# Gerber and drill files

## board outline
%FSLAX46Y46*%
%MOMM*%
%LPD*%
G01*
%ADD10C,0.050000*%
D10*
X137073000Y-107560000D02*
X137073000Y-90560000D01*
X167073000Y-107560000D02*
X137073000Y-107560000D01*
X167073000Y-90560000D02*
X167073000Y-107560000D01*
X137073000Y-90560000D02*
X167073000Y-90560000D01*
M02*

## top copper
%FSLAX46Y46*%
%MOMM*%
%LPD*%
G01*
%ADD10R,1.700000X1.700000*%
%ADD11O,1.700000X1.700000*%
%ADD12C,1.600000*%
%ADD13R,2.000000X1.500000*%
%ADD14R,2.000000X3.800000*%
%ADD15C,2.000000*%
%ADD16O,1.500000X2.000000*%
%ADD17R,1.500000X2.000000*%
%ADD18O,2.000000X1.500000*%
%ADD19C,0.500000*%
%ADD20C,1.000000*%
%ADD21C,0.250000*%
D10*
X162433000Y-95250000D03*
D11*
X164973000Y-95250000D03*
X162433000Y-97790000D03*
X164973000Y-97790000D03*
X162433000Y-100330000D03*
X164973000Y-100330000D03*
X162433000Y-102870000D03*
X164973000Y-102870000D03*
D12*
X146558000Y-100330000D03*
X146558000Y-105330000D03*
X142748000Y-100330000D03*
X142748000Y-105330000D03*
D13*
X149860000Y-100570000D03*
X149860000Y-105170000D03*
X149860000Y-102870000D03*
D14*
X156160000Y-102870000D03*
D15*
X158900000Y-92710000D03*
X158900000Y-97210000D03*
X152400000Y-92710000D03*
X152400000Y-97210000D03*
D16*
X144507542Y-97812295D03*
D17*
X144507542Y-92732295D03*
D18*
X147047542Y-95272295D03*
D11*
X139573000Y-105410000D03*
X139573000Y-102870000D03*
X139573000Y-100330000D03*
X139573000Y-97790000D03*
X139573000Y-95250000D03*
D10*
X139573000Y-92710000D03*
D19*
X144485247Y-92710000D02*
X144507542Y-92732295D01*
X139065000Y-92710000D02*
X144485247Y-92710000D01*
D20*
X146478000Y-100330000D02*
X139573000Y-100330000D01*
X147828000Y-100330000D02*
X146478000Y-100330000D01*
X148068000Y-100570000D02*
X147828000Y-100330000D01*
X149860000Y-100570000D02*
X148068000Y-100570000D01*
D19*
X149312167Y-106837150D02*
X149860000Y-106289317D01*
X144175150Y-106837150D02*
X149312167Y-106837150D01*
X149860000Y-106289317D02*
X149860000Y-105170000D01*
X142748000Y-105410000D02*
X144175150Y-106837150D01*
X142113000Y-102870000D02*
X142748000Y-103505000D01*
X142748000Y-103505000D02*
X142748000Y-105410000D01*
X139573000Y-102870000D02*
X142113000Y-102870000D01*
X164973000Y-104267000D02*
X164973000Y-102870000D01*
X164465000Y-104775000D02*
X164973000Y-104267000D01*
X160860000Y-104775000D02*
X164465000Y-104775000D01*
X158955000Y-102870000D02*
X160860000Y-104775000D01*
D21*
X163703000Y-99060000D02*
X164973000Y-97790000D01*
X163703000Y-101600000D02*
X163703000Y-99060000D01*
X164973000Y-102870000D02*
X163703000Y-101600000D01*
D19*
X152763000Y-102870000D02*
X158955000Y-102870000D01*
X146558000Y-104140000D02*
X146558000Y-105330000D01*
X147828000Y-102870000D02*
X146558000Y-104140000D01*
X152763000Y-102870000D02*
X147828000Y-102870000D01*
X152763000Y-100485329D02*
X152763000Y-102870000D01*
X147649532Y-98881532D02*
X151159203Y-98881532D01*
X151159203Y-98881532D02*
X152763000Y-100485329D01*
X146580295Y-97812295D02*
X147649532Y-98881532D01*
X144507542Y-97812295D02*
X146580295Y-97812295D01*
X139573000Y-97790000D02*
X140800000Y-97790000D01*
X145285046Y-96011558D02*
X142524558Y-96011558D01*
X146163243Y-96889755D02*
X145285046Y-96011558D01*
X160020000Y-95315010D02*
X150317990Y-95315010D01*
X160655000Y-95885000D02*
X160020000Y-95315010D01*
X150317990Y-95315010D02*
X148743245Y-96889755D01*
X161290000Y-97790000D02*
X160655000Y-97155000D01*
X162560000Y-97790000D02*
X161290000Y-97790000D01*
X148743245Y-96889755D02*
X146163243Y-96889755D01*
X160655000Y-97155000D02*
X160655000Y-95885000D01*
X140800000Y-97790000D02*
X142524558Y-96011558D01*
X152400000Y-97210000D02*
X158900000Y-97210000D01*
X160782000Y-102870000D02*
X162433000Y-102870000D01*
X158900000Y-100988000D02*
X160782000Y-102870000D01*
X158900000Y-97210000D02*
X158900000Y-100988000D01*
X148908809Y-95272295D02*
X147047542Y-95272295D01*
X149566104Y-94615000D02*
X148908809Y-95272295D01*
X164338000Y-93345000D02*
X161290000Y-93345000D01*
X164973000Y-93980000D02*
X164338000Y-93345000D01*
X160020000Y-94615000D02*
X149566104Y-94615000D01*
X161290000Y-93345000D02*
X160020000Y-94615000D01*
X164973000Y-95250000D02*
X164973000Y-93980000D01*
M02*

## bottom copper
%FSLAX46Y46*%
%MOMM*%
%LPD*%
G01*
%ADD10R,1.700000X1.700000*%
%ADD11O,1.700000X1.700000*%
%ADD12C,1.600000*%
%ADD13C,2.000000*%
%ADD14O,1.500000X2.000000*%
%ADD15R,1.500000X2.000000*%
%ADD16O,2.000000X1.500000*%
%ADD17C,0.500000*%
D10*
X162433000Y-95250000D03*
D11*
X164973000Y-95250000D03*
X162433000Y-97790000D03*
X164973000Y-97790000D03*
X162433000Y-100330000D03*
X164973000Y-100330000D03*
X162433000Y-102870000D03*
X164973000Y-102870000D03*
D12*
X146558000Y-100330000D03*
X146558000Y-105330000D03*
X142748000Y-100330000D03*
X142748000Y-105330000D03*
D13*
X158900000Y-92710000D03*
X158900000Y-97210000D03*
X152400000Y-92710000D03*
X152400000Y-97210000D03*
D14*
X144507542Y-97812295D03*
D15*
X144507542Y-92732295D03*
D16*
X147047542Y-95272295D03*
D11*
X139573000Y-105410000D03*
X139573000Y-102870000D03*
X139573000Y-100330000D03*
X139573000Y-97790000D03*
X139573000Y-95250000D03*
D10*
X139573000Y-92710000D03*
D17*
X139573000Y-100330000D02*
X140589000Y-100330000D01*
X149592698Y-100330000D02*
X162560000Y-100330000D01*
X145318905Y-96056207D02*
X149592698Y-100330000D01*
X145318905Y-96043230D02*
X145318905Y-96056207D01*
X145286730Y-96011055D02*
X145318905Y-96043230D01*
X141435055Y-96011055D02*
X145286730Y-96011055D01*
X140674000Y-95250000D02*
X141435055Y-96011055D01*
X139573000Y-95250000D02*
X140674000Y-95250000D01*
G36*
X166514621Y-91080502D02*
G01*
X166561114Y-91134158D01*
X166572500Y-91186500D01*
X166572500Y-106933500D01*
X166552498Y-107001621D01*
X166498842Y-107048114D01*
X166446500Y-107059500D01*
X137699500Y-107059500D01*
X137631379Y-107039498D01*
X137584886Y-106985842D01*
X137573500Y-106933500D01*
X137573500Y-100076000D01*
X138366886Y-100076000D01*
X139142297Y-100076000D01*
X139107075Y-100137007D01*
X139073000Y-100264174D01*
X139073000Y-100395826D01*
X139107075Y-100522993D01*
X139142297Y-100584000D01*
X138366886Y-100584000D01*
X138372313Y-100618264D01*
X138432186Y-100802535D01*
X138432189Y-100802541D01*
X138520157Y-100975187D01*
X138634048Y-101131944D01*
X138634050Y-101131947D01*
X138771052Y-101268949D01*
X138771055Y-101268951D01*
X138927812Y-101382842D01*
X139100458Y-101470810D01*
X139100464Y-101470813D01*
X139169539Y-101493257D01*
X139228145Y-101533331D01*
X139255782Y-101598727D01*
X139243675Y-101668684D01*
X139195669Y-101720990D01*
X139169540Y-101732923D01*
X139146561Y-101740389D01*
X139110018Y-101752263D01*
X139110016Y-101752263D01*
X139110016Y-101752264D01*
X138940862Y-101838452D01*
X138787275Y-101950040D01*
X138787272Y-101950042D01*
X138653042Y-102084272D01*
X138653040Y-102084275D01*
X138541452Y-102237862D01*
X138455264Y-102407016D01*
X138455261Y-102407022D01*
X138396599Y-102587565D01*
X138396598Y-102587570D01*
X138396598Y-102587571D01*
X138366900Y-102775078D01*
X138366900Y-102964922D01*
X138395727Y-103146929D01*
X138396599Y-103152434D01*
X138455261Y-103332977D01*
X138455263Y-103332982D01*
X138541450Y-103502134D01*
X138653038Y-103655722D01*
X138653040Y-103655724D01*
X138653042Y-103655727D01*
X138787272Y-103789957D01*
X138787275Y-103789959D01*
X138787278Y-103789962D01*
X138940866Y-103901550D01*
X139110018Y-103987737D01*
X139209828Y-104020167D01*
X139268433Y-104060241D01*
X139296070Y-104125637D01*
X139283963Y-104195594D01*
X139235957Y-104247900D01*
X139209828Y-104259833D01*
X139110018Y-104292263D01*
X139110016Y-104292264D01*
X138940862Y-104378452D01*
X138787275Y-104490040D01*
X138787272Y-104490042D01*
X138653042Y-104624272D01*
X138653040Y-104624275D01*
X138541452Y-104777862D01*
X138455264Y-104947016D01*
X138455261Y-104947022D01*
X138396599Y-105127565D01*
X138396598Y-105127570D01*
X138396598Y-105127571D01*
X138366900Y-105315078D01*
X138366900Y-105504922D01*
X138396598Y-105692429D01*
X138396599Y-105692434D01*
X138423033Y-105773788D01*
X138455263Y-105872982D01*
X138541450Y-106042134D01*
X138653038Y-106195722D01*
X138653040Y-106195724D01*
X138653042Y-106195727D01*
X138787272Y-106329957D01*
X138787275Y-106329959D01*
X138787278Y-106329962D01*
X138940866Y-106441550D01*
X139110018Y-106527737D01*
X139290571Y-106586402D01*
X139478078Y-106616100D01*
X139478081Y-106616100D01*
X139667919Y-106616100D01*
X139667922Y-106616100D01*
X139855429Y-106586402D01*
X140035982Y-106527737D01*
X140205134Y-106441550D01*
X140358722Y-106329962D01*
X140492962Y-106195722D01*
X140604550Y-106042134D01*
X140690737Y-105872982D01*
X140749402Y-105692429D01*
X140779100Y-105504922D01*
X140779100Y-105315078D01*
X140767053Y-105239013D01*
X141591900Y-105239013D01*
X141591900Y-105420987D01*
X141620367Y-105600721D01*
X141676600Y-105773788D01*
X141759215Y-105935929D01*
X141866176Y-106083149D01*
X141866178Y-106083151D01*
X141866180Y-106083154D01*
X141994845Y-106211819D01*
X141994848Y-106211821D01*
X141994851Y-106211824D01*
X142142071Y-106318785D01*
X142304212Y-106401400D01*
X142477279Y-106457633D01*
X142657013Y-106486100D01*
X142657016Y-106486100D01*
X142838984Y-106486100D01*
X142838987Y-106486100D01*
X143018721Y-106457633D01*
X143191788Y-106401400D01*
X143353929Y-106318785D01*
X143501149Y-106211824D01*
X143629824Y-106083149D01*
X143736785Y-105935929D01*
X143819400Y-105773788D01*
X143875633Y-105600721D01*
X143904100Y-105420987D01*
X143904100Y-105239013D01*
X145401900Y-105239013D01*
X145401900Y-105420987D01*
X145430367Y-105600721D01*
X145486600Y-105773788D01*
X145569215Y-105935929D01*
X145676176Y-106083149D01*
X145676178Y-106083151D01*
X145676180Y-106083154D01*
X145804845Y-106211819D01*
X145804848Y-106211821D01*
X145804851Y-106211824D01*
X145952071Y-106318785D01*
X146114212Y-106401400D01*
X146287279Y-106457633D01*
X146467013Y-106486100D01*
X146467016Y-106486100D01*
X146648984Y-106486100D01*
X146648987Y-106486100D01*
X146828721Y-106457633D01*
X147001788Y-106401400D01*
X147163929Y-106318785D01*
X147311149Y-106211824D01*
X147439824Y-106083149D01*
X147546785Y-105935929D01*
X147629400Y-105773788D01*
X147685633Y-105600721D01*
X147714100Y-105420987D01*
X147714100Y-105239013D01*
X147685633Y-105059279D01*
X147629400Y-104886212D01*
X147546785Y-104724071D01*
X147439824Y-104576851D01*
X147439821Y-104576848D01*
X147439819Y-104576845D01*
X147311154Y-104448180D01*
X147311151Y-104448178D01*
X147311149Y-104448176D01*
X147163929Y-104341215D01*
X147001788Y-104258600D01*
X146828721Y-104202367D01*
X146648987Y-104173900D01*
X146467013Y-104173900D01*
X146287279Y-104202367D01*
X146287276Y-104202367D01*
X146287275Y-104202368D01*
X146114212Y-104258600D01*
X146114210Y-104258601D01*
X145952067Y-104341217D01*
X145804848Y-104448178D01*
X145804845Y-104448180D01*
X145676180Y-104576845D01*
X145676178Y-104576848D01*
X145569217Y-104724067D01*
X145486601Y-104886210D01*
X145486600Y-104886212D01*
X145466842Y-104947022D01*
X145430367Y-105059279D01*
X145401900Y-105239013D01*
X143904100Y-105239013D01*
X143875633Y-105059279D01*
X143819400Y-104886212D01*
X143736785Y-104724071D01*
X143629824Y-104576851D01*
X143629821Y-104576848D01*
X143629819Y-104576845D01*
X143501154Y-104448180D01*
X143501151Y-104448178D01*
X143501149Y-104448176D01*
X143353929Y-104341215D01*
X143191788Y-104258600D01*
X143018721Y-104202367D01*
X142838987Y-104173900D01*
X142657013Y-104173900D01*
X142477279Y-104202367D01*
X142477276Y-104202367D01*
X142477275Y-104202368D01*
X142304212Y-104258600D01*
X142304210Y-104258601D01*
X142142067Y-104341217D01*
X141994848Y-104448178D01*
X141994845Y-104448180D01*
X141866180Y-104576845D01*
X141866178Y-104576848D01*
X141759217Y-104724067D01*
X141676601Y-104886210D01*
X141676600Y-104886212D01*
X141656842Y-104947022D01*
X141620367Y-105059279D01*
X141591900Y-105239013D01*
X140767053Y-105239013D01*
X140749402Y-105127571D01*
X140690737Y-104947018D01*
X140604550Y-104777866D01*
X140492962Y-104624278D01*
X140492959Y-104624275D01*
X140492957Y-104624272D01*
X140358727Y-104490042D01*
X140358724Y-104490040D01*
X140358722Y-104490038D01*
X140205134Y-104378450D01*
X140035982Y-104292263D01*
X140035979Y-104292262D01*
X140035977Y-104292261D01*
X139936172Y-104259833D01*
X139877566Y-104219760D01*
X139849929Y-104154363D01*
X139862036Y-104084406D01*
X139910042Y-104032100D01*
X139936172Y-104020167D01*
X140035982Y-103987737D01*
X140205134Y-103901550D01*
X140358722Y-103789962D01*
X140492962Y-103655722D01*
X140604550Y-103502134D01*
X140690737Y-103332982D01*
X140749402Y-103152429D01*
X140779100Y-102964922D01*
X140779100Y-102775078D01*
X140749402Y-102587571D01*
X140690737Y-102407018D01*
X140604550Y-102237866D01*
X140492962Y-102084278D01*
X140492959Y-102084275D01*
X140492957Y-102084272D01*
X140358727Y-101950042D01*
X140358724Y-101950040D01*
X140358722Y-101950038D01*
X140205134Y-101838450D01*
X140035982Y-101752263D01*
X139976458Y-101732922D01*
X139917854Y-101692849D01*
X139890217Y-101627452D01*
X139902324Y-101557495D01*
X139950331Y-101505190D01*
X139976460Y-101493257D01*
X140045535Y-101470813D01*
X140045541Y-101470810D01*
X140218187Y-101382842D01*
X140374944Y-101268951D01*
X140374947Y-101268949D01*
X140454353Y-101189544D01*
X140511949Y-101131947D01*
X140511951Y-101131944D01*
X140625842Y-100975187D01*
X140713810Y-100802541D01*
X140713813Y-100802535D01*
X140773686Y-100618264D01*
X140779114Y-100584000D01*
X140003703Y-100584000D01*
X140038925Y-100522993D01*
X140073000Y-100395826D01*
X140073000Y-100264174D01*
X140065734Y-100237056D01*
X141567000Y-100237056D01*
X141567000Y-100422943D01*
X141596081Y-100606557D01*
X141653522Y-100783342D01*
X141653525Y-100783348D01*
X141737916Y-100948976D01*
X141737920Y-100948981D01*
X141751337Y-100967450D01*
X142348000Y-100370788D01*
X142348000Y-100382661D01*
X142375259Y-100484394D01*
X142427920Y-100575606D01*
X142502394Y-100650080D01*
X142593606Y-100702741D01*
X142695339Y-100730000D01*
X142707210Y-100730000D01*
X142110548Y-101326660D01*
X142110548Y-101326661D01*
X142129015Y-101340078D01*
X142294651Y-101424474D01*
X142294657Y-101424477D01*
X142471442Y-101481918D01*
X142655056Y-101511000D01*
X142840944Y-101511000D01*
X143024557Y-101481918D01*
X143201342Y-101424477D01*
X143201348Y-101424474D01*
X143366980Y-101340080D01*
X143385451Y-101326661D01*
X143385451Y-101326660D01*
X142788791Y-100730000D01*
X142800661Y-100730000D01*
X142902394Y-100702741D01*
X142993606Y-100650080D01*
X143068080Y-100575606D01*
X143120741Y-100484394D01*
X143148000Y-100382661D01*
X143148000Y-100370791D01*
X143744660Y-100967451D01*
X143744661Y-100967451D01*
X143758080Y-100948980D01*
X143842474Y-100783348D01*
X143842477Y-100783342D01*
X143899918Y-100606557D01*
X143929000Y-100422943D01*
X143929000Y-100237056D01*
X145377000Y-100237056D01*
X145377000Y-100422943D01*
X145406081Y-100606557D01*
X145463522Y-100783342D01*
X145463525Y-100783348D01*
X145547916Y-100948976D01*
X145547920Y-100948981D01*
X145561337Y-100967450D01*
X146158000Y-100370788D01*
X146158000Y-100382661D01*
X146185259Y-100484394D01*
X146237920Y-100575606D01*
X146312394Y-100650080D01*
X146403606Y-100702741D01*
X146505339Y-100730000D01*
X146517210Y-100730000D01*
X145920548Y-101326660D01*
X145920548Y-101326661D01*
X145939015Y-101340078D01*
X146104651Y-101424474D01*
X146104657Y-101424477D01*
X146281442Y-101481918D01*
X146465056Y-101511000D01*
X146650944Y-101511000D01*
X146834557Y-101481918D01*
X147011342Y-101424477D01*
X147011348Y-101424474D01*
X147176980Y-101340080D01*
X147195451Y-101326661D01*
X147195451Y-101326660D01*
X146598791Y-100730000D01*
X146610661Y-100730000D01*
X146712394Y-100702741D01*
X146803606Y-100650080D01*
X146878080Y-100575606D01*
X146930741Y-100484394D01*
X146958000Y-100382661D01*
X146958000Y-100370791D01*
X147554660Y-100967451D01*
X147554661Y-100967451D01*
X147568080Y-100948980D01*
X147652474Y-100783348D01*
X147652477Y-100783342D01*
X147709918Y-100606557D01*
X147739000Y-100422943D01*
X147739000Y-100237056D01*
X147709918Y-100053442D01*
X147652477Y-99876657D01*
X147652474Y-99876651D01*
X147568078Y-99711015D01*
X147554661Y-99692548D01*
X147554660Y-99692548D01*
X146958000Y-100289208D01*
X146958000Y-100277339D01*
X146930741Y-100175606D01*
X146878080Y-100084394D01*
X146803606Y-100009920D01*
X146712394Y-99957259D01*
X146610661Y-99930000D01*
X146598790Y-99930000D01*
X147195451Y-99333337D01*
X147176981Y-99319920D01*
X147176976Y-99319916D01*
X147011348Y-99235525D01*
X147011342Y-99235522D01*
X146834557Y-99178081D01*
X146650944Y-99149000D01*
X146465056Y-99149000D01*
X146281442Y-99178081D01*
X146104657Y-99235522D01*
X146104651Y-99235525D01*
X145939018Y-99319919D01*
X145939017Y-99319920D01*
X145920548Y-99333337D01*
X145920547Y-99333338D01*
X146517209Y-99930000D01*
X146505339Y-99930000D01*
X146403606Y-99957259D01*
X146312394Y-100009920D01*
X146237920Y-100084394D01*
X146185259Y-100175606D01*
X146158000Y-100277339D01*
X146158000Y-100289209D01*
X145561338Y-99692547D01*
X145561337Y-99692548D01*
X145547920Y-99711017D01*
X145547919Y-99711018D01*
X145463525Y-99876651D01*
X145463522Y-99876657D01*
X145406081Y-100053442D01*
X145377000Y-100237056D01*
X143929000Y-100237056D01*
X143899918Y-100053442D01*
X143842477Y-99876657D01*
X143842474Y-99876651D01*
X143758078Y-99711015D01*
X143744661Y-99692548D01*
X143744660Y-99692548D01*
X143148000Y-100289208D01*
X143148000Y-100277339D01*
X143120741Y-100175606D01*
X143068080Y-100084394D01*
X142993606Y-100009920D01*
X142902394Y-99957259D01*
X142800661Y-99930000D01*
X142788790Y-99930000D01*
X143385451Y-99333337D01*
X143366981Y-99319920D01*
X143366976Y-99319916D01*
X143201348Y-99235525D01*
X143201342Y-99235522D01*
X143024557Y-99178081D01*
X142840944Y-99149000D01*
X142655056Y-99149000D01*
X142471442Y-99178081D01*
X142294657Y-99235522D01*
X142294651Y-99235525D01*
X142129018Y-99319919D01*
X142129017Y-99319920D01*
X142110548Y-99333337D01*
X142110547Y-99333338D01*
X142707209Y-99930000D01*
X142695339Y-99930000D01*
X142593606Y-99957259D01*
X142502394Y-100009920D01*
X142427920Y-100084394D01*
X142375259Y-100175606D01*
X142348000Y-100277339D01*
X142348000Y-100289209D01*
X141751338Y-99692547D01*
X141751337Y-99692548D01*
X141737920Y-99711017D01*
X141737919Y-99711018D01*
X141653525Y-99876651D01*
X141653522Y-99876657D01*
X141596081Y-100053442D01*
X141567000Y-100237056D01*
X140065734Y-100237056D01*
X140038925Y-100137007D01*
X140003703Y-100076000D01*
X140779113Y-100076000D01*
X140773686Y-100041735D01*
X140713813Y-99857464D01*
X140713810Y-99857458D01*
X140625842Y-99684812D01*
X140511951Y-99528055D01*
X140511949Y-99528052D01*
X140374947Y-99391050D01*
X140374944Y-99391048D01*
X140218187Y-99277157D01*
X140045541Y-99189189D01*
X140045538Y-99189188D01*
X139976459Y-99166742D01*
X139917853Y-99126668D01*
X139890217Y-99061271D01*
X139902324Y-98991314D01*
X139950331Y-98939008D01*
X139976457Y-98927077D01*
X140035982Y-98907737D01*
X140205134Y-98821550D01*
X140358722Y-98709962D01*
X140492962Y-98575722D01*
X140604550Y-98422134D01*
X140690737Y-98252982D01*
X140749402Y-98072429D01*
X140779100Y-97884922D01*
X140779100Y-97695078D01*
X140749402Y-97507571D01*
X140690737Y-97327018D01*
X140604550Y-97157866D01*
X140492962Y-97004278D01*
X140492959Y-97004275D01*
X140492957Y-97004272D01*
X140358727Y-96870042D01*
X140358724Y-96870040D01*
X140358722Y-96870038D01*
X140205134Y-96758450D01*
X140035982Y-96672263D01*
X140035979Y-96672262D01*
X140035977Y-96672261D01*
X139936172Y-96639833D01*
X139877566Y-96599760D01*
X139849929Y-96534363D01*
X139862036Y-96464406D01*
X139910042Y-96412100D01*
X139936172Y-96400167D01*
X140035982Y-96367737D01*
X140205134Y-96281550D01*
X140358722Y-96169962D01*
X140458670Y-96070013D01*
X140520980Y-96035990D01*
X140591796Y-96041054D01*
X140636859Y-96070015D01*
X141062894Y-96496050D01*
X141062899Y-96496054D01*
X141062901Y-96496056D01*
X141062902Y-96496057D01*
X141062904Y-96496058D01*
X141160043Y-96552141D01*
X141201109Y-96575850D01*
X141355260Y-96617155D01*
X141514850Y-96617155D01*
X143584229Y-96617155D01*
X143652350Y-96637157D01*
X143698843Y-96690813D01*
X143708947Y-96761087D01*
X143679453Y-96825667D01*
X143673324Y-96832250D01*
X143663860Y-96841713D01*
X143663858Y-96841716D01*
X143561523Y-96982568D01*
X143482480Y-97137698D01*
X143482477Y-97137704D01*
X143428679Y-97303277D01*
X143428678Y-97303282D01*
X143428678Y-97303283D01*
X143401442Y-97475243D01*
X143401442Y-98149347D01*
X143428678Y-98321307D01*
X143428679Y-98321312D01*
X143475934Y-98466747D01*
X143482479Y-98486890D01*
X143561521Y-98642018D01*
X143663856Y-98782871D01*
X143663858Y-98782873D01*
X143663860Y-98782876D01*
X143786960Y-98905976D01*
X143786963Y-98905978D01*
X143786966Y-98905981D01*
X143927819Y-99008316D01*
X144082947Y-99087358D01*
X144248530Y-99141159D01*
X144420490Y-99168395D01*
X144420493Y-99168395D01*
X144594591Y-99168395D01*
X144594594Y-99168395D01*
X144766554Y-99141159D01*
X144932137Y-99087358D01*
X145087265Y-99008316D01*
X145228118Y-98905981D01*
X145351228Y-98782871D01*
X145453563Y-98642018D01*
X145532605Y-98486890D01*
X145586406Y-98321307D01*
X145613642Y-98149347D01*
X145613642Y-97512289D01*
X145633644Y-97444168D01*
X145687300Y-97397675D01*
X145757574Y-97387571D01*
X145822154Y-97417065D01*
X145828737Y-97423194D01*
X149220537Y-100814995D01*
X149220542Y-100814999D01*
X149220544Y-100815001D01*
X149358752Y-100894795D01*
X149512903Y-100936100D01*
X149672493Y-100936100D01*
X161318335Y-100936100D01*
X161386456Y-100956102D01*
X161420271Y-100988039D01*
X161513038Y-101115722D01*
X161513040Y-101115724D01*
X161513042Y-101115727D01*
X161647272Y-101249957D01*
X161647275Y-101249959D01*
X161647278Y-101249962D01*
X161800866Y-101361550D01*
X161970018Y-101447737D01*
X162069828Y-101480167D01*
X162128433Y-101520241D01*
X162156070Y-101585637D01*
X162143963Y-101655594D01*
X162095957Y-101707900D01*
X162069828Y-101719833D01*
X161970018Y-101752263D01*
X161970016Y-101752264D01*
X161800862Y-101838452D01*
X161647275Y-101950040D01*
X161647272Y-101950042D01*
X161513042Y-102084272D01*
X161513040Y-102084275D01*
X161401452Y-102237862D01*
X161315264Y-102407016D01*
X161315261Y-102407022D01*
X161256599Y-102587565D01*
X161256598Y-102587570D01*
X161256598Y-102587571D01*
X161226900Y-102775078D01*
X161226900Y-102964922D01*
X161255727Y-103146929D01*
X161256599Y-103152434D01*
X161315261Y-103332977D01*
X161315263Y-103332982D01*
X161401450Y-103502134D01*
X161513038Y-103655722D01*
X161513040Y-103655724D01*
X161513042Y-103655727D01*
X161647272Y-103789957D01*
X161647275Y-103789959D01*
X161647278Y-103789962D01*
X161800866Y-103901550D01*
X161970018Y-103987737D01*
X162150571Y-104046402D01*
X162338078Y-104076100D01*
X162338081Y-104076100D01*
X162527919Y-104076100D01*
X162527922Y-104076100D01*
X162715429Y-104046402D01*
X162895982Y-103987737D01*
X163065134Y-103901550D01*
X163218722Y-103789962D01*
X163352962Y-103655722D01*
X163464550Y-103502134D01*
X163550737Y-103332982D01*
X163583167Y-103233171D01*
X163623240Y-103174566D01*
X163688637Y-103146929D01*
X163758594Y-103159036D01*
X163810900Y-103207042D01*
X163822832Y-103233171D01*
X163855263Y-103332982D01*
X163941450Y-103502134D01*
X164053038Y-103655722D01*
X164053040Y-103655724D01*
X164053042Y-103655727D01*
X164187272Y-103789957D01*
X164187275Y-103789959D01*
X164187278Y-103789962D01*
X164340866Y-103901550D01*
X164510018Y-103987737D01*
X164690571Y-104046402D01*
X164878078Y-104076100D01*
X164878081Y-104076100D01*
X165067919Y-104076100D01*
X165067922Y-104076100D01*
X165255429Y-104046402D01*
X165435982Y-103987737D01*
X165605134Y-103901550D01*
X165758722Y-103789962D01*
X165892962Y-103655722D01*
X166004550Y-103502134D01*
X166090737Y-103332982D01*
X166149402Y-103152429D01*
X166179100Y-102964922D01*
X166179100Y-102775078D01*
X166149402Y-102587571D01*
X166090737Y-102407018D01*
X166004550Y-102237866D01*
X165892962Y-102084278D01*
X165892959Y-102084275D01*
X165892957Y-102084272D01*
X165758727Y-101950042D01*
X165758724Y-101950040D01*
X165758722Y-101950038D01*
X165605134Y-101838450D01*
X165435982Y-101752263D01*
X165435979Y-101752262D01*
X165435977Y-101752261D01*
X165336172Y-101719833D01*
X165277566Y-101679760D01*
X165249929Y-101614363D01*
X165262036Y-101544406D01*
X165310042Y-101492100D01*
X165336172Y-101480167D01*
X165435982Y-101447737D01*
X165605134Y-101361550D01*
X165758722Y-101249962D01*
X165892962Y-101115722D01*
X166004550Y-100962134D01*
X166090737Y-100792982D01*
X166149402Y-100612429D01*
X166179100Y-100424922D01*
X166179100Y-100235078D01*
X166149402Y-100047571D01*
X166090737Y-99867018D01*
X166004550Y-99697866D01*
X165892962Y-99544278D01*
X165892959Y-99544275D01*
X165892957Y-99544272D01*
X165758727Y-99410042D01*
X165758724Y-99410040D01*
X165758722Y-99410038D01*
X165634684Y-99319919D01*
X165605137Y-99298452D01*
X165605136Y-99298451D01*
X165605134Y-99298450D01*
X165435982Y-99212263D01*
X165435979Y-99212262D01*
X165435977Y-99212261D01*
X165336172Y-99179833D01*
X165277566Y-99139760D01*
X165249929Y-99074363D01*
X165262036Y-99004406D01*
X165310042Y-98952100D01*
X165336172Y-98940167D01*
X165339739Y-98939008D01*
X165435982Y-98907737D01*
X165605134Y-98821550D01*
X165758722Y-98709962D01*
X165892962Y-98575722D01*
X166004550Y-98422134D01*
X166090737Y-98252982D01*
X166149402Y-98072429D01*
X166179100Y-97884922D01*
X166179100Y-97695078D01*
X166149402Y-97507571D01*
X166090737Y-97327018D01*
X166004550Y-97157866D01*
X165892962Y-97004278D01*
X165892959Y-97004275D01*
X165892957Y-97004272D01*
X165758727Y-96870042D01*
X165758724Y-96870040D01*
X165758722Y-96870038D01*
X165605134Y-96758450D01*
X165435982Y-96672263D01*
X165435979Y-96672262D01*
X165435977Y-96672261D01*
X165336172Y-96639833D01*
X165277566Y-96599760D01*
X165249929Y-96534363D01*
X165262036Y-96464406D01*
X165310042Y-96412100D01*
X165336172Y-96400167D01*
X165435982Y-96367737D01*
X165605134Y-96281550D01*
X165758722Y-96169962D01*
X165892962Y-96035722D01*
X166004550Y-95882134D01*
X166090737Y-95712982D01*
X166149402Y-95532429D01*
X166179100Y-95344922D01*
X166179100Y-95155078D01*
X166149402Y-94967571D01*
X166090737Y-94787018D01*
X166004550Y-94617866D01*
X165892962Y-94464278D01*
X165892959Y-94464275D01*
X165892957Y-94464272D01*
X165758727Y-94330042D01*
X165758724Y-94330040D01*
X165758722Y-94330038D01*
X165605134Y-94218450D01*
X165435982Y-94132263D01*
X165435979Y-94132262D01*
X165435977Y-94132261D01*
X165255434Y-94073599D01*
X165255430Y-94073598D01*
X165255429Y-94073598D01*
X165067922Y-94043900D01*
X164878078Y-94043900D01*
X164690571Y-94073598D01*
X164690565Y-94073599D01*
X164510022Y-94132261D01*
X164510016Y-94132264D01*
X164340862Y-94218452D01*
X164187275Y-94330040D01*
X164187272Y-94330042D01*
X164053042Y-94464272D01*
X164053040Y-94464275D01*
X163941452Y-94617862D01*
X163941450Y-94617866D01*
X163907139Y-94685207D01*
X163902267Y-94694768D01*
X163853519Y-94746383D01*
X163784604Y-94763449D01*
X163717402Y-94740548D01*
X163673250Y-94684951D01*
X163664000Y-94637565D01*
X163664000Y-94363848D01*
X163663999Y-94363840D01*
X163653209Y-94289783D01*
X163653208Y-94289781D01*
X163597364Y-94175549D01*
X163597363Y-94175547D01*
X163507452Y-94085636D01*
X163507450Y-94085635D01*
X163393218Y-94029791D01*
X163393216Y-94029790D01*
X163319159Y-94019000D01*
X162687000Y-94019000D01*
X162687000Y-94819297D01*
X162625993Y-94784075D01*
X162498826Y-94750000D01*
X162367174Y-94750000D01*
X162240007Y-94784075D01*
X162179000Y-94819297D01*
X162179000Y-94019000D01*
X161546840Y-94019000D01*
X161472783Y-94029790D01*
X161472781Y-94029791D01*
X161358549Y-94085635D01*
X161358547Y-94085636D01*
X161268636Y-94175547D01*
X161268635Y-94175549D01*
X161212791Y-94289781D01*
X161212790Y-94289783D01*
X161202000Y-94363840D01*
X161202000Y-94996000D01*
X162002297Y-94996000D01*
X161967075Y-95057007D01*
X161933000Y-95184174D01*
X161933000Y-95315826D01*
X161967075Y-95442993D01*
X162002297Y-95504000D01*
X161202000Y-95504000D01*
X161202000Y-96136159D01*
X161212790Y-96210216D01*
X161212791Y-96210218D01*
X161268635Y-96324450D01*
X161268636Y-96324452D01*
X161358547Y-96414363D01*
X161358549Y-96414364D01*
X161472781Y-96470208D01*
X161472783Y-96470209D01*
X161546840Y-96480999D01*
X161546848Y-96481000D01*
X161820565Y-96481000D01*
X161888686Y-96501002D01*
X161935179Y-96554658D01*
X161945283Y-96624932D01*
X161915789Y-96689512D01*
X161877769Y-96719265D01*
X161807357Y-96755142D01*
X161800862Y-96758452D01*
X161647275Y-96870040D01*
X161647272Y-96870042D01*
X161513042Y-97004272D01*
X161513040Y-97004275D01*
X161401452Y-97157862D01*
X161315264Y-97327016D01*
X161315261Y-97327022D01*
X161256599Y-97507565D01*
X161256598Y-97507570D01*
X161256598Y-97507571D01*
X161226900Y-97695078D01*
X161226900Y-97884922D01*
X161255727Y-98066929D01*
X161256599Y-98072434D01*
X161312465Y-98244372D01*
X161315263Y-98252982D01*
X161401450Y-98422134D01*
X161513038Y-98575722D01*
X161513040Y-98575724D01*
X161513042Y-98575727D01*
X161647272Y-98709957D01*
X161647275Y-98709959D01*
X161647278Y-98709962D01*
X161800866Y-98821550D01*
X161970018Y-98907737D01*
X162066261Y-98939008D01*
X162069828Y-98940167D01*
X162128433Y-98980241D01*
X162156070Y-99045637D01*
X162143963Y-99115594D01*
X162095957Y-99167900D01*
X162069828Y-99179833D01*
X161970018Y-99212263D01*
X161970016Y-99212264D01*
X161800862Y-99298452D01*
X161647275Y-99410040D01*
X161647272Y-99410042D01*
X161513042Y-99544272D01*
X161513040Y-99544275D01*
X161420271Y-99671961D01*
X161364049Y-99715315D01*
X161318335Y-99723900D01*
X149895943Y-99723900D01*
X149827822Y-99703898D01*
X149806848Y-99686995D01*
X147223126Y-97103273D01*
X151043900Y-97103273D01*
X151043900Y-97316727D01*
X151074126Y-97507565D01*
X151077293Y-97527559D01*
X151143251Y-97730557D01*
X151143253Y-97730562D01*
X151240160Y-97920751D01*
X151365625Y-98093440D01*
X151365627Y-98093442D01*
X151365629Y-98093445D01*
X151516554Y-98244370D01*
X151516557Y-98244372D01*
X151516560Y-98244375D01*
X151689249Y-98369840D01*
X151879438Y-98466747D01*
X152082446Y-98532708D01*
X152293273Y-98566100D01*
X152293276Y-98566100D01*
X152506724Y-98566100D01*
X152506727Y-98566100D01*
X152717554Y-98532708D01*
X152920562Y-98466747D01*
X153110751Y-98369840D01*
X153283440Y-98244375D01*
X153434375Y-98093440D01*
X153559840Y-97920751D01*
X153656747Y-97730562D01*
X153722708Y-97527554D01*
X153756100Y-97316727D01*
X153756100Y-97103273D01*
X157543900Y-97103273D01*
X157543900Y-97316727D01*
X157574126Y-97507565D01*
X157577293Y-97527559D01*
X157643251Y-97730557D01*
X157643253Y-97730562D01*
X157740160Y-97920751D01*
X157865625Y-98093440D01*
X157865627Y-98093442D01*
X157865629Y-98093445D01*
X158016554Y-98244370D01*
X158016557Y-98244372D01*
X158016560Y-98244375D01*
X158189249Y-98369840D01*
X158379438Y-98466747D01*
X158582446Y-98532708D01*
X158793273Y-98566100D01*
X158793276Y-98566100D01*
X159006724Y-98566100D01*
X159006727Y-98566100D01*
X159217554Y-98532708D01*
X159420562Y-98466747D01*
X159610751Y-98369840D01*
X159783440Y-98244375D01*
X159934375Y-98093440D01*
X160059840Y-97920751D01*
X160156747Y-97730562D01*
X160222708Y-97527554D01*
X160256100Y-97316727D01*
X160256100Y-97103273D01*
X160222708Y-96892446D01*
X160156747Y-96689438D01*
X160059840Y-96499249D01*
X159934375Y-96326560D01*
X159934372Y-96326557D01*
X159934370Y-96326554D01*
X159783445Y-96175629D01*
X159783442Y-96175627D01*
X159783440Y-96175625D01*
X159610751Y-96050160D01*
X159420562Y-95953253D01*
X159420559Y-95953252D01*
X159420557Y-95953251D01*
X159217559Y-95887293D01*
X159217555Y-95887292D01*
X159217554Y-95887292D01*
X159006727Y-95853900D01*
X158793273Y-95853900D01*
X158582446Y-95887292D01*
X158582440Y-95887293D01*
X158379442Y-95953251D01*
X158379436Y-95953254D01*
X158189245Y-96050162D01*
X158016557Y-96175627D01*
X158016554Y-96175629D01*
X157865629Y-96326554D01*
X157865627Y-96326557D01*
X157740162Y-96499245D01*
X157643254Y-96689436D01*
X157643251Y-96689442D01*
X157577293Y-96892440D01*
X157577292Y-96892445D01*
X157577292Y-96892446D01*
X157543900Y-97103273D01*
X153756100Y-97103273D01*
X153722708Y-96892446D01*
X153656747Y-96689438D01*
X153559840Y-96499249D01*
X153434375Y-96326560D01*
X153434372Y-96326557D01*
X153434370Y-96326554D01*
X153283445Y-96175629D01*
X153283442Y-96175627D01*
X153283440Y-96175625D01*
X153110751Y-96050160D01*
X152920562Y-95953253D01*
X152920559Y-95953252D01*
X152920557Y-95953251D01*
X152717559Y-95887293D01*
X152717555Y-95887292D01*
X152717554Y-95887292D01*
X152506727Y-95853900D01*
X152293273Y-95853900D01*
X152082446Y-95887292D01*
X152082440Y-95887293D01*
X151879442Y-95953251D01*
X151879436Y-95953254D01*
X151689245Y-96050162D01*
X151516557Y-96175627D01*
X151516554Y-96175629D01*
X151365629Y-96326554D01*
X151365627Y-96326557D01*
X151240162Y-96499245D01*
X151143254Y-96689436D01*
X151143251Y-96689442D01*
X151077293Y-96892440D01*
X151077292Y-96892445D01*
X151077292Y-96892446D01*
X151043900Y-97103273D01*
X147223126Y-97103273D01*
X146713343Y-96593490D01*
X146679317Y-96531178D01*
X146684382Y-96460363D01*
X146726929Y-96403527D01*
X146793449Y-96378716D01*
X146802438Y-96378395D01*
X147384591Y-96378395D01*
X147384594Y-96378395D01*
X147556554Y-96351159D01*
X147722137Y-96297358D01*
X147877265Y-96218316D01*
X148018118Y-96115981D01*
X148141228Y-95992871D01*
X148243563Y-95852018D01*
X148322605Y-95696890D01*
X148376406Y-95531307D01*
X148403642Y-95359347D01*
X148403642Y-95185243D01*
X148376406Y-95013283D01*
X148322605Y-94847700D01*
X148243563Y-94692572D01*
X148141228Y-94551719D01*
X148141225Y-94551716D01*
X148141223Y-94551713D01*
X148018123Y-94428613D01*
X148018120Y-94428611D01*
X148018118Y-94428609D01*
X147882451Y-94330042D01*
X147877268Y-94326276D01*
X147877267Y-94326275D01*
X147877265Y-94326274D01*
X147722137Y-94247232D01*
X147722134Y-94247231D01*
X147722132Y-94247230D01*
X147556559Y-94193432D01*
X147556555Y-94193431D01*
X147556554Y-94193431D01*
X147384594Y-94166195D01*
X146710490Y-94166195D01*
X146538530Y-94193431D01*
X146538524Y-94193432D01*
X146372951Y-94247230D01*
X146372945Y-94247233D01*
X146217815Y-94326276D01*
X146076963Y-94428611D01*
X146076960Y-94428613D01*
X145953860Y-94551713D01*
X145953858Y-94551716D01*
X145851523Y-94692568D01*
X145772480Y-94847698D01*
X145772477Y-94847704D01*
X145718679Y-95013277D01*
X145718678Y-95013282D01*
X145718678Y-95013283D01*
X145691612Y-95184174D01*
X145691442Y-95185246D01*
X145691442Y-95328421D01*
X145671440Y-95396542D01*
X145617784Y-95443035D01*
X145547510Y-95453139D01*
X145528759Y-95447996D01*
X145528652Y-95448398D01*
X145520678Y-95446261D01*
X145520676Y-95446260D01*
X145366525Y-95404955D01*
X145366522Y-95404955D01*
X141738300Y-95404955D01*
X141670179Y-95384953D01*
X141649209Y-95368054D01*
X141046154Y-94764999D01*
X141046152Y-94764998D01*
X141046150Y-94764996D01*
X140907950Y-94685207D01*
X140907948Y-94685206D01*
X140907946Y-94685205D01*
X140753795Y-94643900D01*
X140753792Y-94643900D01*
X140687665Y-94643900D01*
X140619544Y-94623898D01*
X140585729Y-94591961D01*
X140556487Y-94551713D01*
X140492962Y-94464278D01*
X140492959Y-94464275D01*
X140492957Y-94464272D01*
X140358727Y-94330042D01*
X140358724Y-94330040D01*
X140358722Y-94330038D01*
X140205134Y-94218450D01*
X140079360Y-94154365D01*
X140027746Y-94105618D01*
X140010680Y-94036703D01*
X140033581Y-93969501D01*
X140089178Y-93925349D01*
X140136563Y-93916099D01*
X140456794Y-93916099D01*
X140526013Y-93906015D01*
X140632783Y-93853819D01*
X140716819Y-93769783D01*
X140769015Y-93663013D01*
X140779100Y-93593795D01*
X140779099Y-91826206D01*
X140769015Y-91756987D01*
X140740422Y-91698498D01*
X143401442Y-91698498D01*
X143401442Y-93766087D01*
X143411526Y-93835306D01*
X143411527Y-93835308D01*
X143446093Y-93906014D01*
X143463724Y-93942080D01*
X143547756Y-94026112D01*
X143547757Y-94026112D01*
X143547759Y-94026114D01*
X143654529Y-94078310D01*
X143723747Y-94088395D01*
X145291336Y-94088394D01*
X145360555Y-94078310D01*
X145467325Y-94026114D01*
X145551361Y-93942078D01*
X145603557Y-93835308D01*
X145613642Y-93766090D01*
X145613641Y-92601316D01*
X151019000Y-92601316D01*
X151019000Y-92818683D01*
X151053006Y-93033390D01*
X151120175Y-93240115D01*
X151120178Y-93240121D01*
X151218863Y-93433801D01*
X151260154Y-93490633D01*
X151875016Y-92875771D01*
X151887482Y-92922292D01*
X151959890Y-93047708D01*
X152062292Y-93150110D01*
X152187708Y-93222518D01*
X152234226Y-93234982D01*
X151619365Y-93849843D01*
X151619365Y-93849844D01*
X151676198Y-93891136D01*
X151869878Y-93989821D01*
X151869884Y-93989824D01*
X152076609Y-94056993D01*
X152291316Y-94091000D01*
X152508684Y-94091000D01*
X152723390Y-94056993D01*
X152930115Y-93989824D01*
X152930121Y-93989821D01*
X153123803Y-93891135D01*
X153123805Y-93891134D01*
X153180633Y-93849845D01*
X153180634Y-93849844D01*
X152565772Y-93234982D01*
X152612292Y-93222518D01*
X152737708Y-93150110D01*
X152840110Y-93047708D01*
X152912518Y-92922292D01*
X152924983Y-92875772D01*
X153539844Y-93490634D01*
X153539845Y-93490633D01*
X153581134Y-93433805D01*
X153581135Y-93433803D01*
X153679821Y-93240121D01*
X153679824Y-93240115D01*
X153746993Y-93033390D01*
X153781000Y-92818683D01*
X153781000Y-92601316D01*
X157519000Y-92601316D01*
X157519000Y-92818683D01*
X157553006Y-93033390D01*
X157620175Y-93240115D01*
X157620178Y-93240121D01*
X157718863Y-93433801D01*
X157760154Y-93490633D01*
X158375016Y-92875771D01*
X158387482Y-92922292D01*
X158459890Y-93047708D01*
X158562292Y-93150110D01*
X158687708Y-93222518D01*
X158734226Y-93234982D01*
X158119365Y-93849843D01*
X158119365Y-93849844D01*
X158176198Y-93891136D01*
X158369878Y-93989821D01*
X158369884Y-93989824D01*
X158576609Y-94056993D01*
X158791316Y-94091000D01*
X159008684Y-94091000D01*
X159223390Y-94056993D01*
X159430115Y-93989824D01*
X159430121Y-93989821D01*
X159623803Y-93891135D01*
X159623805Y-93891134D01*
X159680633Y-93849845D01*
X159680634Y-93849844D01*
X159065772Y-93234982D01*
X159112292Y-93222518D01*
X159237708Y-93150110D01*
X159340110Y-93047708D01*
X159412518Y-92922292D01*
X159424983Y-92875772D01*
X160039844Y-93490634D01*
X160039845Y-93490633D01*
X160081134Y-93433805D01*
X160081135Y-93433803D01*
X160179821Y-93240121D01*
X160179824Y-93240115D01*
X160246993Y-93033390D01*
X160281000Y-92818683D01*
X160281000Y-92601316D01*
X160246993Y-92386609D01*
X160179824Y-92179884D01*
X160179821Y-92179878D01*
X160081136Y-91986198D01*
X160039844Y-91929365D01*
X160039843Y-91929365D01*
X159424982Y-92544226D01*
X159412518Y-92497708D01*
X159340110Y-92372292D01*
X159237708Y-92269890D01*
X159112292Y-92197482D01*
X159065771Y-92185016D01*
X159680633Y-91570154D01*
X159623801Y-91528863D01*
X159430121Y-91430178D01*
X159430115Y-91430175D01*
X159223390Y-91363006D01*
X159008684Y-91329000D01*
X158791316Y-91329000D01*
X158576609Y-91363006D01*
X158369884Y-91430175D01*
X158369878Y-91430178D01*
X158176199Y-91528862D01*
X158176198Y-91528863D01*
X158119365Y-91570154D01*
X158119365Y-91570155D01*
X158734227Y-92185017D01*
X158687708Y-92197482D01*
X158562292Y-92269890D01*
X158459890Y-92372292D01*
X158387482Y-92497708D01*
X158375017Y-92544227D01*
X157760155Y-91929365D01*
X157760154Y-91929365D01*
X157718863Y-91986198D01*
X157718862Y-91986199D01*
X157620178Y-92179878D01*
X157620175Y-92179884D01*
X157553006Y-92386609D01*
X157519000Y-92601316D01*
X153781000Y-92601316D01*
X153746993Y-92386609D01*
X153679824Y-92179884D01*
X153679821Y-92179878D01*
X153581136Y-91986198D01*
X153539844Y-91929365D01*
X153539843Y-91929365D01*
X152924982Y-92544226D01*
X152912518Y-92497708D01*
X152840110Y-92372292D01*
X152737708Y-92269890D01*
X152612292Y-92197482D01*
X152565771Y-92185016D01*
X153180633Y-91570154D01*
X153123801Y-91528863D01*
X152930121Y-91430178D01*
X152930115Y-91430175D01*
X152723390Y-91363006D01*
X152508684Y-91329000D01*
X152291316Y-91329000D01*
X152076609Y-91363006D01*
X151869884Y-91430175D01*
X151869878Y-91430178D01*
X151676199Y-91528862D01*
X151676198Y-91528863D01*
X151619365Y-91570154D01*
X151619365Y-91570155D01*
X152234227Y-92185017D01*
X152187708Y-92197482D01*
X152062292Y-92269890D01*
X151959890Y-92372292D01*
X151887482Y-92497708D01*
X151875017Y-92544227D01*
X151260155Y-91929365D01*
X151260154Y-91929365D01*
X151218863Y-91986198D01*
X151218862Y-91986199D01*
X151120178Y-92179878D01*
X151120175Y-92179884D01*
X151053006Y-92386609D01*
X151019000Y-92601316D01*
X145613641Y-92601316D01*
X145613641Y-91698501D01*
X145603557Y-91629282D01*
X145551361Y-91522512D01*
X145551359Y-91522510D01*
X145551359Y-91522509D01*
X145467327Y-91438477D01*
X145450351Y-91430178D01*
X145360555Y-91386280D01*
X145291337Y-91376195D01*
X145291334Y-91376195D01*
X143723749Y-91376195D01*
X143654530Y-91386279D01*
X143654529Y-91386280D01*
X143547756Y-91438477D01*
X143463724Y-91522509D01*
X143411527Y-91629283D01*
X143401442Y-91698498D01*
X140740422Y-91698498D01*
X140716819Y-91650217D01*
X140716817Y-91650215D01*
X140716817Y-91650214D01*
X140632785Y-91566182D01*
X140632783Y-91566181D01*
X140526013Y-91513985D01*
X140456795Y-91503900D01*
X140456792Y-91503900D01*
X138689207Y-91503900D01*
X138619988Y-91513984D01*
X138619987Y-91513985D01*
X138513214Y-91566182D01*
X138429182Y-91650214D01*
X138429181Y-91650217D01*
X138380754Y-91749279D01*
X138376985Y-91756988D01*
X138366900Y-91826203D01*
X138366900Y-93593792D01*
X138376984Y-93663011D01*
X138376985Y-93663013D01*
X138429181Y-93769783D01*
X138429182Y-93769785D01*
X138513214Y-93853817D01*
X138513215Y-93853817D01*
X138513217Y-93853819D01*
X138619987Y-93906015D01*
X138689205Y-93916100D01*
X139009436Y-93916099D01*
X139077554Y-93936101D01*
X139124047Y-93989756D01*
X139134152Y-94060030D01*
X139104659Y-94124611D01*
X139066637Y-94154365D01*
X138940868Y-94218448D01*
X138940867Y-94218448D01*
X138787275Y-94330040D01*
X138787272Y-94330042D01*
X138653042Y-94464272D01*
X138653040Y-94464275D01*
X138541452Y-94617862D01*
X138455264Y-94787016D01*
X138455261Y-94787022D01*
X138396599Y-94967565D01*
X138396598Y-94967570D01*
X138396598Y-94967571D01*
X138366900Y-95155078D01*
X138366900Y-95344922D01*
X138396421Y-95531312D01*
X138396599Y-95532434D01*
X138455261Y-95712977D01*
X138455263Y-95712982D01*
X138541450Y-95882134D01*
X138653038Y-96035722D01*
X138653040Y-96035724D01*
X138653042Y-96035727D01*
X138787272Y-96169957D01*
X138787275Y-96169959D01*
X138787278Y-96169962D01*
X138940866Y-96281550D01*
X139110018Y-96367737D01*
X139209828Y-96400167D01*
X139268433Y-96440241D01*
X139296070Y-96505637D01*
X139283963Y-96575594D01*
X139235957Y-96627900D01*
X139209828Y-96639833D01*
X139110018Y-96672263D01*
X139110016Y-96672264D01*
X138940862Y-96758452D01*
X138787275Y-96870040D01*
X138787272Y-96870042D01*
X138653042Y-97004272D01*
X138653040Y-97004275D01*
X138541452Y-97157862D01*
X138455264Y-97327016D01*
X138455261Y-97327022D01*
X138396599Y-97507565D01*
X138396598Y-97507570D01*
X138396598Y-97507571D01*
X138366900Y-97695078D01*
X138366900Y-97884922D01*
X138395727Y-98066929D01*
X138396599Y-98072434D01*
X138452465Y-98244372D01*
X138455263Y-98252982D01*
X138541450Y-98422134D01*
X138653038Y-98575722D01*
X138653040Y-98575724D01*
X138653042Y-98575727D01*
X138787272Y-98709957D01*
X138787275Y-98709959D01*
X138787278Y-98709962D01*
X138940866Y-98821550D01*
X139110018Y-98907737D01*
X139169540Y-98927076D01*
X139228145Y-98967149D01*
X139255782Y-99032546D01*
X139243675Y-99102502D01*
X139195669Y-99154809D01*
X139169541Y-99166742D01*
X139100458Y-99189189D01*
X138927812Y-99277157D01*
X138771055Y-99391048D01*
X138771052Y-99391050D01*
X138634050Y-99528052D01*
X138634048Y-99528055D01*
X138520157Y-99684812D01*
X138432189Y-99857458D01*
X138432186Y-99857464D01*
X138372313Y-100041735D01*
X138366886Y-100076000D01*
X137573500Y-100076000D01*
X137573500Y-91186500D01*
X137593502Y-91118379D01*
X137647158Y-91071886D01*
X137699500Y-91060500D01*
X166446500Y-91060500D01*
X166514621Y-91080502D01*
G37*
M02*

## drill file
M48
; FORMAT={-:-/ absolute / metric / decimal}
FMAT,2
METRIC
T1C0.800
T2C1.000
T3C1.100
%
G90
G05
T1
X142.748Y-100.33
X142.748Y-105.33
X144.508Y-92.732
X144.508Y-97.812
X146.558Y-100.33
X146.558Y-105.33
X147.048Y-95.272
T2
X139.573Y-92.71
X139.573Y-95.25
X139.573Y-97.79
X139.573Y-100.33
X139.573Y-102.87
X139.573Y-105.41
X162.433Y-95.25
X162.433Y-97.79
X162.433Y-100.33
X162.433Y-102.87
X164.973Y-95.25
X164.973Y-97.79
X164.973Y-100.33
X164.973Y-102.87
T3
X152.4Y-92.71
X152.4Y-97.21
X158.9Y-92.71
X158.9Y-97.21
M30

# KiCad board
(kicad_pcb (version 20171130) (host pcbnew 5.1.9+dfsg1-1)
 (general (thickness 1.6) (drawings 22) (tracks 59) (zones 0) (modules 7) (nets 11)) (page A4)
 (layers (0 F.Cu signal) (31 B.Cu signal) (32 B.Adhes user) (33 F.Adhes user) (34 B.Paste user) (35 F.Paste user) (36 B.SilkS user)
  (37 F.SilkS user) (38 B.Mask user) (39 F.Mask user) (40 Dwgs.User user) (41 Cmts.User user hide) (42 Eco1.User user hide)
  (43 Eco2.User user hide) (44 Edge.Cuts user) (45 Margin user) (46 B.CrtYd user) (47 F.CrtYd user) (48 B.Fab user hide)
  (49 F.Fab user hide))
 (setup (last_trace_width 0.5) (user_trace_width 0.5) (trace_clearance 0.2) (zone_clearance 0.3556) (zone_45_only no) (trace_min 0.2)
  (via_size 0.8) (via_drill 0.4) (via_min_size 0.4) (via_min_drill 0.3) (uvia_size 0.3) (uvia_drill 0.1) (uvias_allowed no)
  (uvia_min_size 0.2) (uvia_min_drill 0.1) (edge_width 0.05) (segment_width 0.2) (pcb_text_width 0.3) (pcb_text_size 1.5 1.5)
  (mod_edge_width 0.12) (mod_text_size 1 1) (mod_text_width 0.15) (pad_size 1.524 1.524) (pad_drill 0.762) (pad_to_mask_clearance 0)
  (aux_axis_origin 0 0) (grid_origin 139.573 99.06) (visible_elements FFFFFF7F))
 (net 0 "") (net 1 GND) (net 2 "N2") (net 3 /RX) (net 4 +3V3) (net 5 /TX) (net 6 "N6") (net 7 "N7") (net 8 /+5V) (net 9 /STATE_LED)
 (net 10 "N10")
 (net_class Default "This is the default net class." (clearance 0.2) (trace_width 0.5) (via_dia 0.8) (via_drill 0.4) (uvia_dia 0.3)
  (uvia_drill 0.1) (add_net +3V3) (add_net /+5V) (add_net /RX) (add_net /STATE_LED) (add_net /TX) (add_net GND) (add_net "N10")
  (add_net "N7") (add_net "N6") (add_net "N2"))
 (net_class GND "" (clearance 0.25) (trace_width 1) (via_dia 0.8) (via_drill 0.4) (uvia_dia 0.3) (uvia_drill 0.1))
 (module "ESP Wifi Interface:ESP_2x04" (layer B.Cu) (at 163.703 99.06 270)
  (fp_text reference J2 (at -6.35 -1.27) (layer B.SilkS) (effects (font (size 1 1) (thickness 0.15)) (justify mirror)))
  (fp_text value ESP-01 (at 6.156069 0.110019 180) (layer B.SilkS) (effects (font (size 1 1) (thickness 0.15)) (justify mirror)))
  (pad 1 thru_hole rect (at -3.81 1.27 180) (size 1.7 1.7) (drill 1) (layers *.Cu *.Mask) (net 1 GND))
  (pad 8 thru_hole oval (at -3.81 -1.27 180) (size 1.7 1.7) (drill 1) (layers *.Cu *.Mask) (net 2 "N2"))
  (pad 2 thru_hole oval (at -1.27 1.27 180) (size 1.7 1.7) (drill 1) (layers *.Cu *.Mask) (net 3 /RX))
  (pad 7 thru_hole oval (at -1.27 -1.27 180) (size 1.7 1.7) (drill 1) (layers *.Cu *.Mask) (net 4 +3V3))
  (pad 3 thru_hole oval (at 1.27 1.27 180) (size 1.7 1.7) (drill 1) (layers *.Cu *.Mask) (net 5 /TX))
  (pad 6 thru_hole oval (at 1.27 -1.27 180) (size 1.7 1.7) (drill 1) (layers *.Cu *.Mask) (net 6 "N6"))
  (pad 4 thru_hole oval (at 3.81 1.27 180) (size 1.7 1.7) (drill 1) (layers *.Cu *.Mask) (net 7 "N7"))
  (pad 5 thru_hole oval (at 3.81 -1.27 180) (size 1.7 1.7) (drill 1) (layers *.Cu *.Mask) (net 4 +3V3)))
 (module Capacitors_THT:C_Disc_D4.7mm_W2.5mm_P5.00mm (layer F.Cu) (at 146.558 105.33 90)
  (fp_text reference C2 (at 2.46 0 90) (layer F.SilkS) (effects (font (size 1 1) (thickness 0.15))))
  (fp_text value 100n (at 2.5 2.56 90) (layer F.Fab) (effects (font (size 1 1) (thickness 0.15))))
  (pad 2 thru_hole circle (at 5 0 90) (size 1.6 1.6) (drill 0.8) (layers *.Cu *.Mask) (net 1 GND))
  (pad 1 thru_hole circle (at 0 0 90) (size 1.6 1.6) (drill 0.8) (layers *.Cu *.Mask) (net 4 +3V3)))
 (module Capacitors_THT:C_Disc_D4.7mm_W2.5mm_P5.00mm (layer F.Cu) (at 142.748 105.33 90)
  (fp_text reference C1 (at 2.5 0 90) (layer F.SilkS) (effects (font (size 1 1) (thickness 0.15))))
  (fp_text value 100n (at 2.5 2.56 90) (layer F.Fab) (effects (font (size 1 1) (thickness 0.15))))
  (pad 2 thru_hole circle (at 5 0 90) (size 1.6 1.6) (drill 0.8) (layers *.Cu *.Mask) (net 1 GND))
  (pad 1 thru_hole circle (at 0 0 90) (size 1.6 1.6) (drill 0.8) (layers *.Cu *.Mask) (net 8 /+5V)))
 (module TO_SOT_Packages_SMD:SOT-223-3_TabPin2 (layer F.Cu) (at 153.01 102.87)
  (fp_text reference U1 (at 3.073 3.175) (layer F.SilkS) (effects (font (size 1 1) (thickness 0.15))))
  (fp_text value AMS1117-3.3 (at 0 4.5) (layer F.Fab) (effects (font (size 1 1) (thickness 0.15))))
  (pad 1 smd rect (at -3.15 -2.3) (size 2 1.5) (layers F.Cu F.Paste F.Mask) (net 1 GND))
  (pad 3 smd rect (at -3.15 2.3) (size 2 1.5) (layers F.Cu F.Paste F.Mask) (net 8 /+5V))
  (pad 2 smd rect (at -3.15 0) (size 2 1.5) (layers F.Cu F.Paste F.Mask) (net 4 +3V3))
  (pad 2 smd rect (at 3.15 0) (size 2 3.8) (layers F.Cu F.Paste F.Mask) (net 4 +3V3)))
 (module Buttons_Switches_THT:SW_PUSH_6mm (layer F.Cu) (at 152.4 92.71)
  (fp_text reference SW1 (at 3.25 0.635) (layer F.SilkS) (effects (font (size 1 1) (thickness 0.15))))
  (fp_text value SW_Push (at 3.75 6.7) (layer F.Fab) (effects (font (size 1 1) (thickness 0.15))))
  (pad 1 thru_hole circle (at 6.5 0 90) (size 2 2) (drill 1.1) (layers *.Cu *.Mask) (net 1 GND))
  (pad 2 thru_hole circle (at 6.5 4.5 90) (size 2 2) (drill 1.1) (layers *.Cu *.Mask) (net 7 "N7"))
  (pad 1 thru_hole circle (at 0 0 90) (size 2 2) (drill 1.1) (layers *.Cu *.Mask) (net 1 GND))
  (pad 2 thru_hole circle (at 0 4.5 90) (size 2 2) (drill 1.1) (layers *.Cu *.Mask) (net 7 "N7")))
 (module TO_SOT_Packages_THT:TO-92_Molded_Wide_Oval (layer F.Cu) (at 144.507542 92.732295 270)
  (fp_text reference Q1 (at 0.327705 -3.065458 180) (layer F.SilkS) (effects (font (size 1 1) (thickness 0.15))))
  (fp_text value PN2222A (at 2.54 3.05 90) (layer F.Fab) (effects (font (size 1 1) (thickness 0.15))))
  (pad 3 thru_hole oval (at 5.08 0) (size 1.5 2) (drill 0.8) (layers *.Cu *.Mask) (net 4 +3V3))
  (pad 1 thru_hole rect (at 0 0) (size 1.5 2) (drill 0.8) (layers *.Cu *.Mask) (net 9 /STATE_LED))
  (pad 2 thru_hole oval (at 2.54 -2.54) (size 2 1.5) (drill 0.8) (layers *.Cu *.Mask) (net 2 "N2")))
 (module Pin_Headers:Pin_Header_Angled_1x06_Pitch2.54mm (layer B.Cu) (at 139.573 92.71 180)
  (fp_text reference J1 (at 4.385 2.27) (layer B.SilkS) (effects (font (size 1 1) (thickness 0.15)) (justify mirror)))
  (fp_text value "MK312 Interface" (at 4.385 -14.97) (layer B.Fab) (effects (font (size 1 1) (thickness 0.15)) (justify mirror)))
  (pad 6 thru_hole oval (at 0 -12.7 180) (size 1.7 1.7) (drill 1) (layers *.Cu *.Mask) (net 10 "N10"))
  (pad 5 thru_hole oval (at 0 -10.16 180) (size 1.7 1.7) (drill 1) (layers *.Cu *.Mask) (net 8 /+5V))
  (pad 4 thru_hole oval (at 0 -7.62 180) (size 1.7 1.7) (drill 1) (layers *.Cu *.Mask) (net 1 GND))
  (pad 3 thru_hole oval (at 0 -5.08 180) (size 1.7 1.7) (drill 1) (layers *.Cu *.Mask) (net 3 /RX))
  (pad 2 thru_hole oval (at 0 -2.54 180) (size 1.7 1.7) (drill 1) (layers *.Cu *.Mask) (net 5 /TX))
  (pad 1 thru_hole rect (at 0 0 180) (size 1.7 1.7) (drill 1) (layers *.Cu *.Mask) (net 9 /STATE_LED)))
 (gr_line (start 137.073 107.56) (end 137.073 90.56) (layer Edge.Cuts) (width 0.05))
 (gr_line (start 167.073 107.56) (end 137.073 107.56) (layer Edge.Cuts) (width 0.05))
 (gr_line (start 167.073 90.56) (end 167.073 107.56) (layer Edge.Cuts) (width 0.05))
 (gr_line (start 137.073 90.56) (end 167.073 90.56) (layer Edge.Cuts) (width 0.05))
 (segment (start 144.485247 92.71) (end 144.507542 92.732295) (width 0.5) (layer F.Cu) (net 9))
 (segment (start 139.065 92.71) (end 144.485247 92.71) (width 0.5) (layer F.Cu) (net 9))
 (segment (start 139.573 100.33) (end 140.589 100.33) (width 0.5) (layer B.Cu) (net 1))
 (segment (start 146.478 100.33) (end 139.573 100.33) (width 1) (layer F.Cu) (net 1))
 (segment (start 147.828 100.33) (end 146.478 100.33) (width 1) (layer F.Cu) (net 1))
 (segment (start 148.068 100.57) (end 147.828 100.33) (width 1) (layer F.Cu) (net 1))
 (segment (start 149.86 100.57) (end 148.068 100.57) (width 1) (layer F.Cu) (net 1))
 (segment (start 149.312167 106.83715) (end 149.86 106.289317) (width 0.5) (layer F.Cu) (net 8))
 (segment (start 144.17515 106.83715) (end 149.312167 106.83715) (width 0.5) (layer F.Cu) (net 8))
 (segment (start 149.86 106.289317) (end 149.86 105.17) (width 0.5) (layer F.Cu) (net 8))
 (segment (start 142.748 105.41) (end 144.17515 106.83715) (width 0.5) (layer F.Cu) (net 8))
 (segment (start 142.113 102.87) (end 142.748 103.505) (width 0.5) (layer F.Cu) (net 8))
 (segment (start 142.748 103.505) (end 142.748 105.41) (width 0.5) (layer F.Cu) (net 8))
 (segment (start 139.573 102.87) (end 142.113 102.87) (width 0.5) (layer F.Cu) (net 8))
 (segment (start 164.973 104.267) (end 164.973 102.87) (width 0.5) (layer F.Cu) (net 4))
 (segment (start 164.465 104.775) (end 164.973 104.267) (width 0.5) (layer F.Cu) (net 4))
 (segment (start 160.86 104.775) (end 164.465 104.775) (width 0.5) (layer F.Cu) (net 4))
 (segment (start 158.955 102.87) (end 160.86 104.775) (width 0.5) (layer F.Cu) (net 4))
 (segment (start 163.703 99.06) (end 164.973 97.79) (width 0.25) (layer F.Cu) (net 4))
 (segment (start 163.703 101.6) (end 163.703 99.06) (width 0.25) (layer F.Cu) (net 4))
 (segment (start 164.973 102.87) (end 163.703 101.6) (width 0.25) (layer F.Cu) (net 4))
 (segment (start 152.763 102.87) (end 158.955 102.87) (width 0.5) (layer F.Cu) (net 4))
 (segment (start 146.558 104.14) (end 146.558 105.33) (width 0.5) (layer F.Cu) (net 4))
 (segment (start 147.828 102.87) (end 146.558 104.14) (width 0.5) (layer F.Cu) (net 4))
 (segment (start 152.763 102.87) (end 147.828 102.87) (width 0.5) (layer F.Cu) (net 4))
 (segment (start 152.763 100.485329) (end 152.763 102.87) (width 0.5) (layer F.Cu) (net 4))
 (segment (start 147.649532 98.881532) (end 151.159203 98.881532) (width 0.5) (layer F.Cu) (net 4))
 (segment (start 151.159203 98.881532) (end 152.763 100.485329) (width 0.5) (layer F.Cu) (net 4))
 (segment (start 146.580295 97.812295) (end 147.649532 98.881532) (width 0.5) (layer F.Cu) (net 4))
 (segment (start 144.507542 97.812295) (end 146.580295 97.812295) (width 0.5) (layer F.Cu) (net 4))
 (segment (start 139.573 97.79) (end 140.8 97.79) (width 0.5) (layer F.Cu) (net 3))
 (segment (start 145.285046 96.011558) (end 142.524558 96.011558) (width 0.5) (layer F.Cu) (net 3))
 (segment (start 146.163243 96.889755) (end 145.285046 96.011558) (width 0.5) (layer F.Cu) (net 3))
 (segment (start 160.02 95.31501) (end 150.31799 95.31501) (width 0.5) (layer F.Cu) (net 3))
 (segment (start 160.655 95.885) (end 160.02 95.31501) (width 0.5) (layer F.Cu) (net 3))
 (segment (start 150.31799 95.31501) (end 148.743245 96.889755) (width 0.5) (layer F.Cu) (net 3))
 (segment (start 161.29 97.79) (end 160.655 97.155) (width 0.5) (layer F.Cu) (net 3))
 (segment (start 162.56 97.79) (end 161.29 97.79) (width 0.5) (layer F.Cu) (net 3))
 (segment (start 148.743245 96.889755) (end 146.163243 96.889755) (width 0.5) (layer F.Cu) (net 3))
 (segment (start 160.655 97.155) (end 160.655 95.885) (width 0.5) (layer F.Cu) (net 3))
 (segment (start 140.8 97.79) (end 142.524558 96.011558) (width 0.5) (layer F.Cu) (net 3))
 (segment (start 149.592698 100.33) (end 162.56 100.33) (width 0.5) (layer B.Cu) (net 5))
 (segment (start 145.318905 96.056207) (end 149.592698 100.33) (width 0.5) (layer B.Cu) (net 5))
 (segment (start 145.318905 96.04323) (end 145.318905 96.056207) (width 0.5) (layer B.Cu) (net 5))
 (segment (start 145.28673 96.011055) (end 145.318905 96.04323) (width 0.5) (layer B.Cu) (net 5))
 (segment (start 141.435055 96.011055) (end 145.28673 96.011055) (width 0.5) (layer B.Cu) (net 5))
 (segment (start 140.674 95.25) (end 141.435055 96.011055) (width 0.5) (layer B.Cu) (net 5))
 (segment (start 139.573 95.25) (end 140.674 95.25) (width 0.5) (layer B.Cu) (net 5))
 (segment (start 152.4 97.21) (end 158.9 97.21) (width 0.5) (layer F.Cu) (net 7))
 (segment (start 160.782 102.87) (end 162.433 102.87) (width 0.5) (layer F.Cu) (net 7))
 (segment (start 158.9 100.988) (end 160.782 102.87) (width 0.5) (layer F.Cu) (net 7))
 (segment (start 158.9 97.21) (end 158.9 100.988) (width 0.5) (layer F.Cu) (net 7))
 (segment (start 148.908809 95.272295) (end 147.047542 95.272295) (width 0.5) (layer F.Cu) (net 2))
 (segment (start 149.566104 94.615) (end 148.908809 95.272295) (width 0.5) (layer F.Cu) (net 2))
 (segment (start 164.338 93.345) (end 161.29 93.345) (width 0.5) (layer F.Cu) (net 2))
 (segment (start 164.973 93.98) (end 164.338 93.345) (width 0.5) (layer F.Cu) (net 2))
 (segment (start 160.02 94.615) (end 149.566104 94.615) (width 0.5) (layer F.Cu) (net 2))
 (segment (start 161.29 93.345) (end 160.02 94.615) (width 0.5) (layer F.Cu) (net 2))
 (segment (start 164.973 95.25) (end 164.973 93.98) (width 0.5) (layer F.Cu) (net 2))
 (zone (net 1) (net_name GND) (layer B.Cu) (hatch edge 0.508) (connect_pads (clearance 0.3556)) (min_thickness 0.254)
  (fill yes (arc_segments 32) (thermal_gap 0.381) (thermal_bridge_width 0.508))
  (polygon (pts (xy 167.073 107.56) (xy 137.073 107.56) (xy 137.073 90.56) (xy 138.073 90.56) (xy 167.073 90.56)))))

